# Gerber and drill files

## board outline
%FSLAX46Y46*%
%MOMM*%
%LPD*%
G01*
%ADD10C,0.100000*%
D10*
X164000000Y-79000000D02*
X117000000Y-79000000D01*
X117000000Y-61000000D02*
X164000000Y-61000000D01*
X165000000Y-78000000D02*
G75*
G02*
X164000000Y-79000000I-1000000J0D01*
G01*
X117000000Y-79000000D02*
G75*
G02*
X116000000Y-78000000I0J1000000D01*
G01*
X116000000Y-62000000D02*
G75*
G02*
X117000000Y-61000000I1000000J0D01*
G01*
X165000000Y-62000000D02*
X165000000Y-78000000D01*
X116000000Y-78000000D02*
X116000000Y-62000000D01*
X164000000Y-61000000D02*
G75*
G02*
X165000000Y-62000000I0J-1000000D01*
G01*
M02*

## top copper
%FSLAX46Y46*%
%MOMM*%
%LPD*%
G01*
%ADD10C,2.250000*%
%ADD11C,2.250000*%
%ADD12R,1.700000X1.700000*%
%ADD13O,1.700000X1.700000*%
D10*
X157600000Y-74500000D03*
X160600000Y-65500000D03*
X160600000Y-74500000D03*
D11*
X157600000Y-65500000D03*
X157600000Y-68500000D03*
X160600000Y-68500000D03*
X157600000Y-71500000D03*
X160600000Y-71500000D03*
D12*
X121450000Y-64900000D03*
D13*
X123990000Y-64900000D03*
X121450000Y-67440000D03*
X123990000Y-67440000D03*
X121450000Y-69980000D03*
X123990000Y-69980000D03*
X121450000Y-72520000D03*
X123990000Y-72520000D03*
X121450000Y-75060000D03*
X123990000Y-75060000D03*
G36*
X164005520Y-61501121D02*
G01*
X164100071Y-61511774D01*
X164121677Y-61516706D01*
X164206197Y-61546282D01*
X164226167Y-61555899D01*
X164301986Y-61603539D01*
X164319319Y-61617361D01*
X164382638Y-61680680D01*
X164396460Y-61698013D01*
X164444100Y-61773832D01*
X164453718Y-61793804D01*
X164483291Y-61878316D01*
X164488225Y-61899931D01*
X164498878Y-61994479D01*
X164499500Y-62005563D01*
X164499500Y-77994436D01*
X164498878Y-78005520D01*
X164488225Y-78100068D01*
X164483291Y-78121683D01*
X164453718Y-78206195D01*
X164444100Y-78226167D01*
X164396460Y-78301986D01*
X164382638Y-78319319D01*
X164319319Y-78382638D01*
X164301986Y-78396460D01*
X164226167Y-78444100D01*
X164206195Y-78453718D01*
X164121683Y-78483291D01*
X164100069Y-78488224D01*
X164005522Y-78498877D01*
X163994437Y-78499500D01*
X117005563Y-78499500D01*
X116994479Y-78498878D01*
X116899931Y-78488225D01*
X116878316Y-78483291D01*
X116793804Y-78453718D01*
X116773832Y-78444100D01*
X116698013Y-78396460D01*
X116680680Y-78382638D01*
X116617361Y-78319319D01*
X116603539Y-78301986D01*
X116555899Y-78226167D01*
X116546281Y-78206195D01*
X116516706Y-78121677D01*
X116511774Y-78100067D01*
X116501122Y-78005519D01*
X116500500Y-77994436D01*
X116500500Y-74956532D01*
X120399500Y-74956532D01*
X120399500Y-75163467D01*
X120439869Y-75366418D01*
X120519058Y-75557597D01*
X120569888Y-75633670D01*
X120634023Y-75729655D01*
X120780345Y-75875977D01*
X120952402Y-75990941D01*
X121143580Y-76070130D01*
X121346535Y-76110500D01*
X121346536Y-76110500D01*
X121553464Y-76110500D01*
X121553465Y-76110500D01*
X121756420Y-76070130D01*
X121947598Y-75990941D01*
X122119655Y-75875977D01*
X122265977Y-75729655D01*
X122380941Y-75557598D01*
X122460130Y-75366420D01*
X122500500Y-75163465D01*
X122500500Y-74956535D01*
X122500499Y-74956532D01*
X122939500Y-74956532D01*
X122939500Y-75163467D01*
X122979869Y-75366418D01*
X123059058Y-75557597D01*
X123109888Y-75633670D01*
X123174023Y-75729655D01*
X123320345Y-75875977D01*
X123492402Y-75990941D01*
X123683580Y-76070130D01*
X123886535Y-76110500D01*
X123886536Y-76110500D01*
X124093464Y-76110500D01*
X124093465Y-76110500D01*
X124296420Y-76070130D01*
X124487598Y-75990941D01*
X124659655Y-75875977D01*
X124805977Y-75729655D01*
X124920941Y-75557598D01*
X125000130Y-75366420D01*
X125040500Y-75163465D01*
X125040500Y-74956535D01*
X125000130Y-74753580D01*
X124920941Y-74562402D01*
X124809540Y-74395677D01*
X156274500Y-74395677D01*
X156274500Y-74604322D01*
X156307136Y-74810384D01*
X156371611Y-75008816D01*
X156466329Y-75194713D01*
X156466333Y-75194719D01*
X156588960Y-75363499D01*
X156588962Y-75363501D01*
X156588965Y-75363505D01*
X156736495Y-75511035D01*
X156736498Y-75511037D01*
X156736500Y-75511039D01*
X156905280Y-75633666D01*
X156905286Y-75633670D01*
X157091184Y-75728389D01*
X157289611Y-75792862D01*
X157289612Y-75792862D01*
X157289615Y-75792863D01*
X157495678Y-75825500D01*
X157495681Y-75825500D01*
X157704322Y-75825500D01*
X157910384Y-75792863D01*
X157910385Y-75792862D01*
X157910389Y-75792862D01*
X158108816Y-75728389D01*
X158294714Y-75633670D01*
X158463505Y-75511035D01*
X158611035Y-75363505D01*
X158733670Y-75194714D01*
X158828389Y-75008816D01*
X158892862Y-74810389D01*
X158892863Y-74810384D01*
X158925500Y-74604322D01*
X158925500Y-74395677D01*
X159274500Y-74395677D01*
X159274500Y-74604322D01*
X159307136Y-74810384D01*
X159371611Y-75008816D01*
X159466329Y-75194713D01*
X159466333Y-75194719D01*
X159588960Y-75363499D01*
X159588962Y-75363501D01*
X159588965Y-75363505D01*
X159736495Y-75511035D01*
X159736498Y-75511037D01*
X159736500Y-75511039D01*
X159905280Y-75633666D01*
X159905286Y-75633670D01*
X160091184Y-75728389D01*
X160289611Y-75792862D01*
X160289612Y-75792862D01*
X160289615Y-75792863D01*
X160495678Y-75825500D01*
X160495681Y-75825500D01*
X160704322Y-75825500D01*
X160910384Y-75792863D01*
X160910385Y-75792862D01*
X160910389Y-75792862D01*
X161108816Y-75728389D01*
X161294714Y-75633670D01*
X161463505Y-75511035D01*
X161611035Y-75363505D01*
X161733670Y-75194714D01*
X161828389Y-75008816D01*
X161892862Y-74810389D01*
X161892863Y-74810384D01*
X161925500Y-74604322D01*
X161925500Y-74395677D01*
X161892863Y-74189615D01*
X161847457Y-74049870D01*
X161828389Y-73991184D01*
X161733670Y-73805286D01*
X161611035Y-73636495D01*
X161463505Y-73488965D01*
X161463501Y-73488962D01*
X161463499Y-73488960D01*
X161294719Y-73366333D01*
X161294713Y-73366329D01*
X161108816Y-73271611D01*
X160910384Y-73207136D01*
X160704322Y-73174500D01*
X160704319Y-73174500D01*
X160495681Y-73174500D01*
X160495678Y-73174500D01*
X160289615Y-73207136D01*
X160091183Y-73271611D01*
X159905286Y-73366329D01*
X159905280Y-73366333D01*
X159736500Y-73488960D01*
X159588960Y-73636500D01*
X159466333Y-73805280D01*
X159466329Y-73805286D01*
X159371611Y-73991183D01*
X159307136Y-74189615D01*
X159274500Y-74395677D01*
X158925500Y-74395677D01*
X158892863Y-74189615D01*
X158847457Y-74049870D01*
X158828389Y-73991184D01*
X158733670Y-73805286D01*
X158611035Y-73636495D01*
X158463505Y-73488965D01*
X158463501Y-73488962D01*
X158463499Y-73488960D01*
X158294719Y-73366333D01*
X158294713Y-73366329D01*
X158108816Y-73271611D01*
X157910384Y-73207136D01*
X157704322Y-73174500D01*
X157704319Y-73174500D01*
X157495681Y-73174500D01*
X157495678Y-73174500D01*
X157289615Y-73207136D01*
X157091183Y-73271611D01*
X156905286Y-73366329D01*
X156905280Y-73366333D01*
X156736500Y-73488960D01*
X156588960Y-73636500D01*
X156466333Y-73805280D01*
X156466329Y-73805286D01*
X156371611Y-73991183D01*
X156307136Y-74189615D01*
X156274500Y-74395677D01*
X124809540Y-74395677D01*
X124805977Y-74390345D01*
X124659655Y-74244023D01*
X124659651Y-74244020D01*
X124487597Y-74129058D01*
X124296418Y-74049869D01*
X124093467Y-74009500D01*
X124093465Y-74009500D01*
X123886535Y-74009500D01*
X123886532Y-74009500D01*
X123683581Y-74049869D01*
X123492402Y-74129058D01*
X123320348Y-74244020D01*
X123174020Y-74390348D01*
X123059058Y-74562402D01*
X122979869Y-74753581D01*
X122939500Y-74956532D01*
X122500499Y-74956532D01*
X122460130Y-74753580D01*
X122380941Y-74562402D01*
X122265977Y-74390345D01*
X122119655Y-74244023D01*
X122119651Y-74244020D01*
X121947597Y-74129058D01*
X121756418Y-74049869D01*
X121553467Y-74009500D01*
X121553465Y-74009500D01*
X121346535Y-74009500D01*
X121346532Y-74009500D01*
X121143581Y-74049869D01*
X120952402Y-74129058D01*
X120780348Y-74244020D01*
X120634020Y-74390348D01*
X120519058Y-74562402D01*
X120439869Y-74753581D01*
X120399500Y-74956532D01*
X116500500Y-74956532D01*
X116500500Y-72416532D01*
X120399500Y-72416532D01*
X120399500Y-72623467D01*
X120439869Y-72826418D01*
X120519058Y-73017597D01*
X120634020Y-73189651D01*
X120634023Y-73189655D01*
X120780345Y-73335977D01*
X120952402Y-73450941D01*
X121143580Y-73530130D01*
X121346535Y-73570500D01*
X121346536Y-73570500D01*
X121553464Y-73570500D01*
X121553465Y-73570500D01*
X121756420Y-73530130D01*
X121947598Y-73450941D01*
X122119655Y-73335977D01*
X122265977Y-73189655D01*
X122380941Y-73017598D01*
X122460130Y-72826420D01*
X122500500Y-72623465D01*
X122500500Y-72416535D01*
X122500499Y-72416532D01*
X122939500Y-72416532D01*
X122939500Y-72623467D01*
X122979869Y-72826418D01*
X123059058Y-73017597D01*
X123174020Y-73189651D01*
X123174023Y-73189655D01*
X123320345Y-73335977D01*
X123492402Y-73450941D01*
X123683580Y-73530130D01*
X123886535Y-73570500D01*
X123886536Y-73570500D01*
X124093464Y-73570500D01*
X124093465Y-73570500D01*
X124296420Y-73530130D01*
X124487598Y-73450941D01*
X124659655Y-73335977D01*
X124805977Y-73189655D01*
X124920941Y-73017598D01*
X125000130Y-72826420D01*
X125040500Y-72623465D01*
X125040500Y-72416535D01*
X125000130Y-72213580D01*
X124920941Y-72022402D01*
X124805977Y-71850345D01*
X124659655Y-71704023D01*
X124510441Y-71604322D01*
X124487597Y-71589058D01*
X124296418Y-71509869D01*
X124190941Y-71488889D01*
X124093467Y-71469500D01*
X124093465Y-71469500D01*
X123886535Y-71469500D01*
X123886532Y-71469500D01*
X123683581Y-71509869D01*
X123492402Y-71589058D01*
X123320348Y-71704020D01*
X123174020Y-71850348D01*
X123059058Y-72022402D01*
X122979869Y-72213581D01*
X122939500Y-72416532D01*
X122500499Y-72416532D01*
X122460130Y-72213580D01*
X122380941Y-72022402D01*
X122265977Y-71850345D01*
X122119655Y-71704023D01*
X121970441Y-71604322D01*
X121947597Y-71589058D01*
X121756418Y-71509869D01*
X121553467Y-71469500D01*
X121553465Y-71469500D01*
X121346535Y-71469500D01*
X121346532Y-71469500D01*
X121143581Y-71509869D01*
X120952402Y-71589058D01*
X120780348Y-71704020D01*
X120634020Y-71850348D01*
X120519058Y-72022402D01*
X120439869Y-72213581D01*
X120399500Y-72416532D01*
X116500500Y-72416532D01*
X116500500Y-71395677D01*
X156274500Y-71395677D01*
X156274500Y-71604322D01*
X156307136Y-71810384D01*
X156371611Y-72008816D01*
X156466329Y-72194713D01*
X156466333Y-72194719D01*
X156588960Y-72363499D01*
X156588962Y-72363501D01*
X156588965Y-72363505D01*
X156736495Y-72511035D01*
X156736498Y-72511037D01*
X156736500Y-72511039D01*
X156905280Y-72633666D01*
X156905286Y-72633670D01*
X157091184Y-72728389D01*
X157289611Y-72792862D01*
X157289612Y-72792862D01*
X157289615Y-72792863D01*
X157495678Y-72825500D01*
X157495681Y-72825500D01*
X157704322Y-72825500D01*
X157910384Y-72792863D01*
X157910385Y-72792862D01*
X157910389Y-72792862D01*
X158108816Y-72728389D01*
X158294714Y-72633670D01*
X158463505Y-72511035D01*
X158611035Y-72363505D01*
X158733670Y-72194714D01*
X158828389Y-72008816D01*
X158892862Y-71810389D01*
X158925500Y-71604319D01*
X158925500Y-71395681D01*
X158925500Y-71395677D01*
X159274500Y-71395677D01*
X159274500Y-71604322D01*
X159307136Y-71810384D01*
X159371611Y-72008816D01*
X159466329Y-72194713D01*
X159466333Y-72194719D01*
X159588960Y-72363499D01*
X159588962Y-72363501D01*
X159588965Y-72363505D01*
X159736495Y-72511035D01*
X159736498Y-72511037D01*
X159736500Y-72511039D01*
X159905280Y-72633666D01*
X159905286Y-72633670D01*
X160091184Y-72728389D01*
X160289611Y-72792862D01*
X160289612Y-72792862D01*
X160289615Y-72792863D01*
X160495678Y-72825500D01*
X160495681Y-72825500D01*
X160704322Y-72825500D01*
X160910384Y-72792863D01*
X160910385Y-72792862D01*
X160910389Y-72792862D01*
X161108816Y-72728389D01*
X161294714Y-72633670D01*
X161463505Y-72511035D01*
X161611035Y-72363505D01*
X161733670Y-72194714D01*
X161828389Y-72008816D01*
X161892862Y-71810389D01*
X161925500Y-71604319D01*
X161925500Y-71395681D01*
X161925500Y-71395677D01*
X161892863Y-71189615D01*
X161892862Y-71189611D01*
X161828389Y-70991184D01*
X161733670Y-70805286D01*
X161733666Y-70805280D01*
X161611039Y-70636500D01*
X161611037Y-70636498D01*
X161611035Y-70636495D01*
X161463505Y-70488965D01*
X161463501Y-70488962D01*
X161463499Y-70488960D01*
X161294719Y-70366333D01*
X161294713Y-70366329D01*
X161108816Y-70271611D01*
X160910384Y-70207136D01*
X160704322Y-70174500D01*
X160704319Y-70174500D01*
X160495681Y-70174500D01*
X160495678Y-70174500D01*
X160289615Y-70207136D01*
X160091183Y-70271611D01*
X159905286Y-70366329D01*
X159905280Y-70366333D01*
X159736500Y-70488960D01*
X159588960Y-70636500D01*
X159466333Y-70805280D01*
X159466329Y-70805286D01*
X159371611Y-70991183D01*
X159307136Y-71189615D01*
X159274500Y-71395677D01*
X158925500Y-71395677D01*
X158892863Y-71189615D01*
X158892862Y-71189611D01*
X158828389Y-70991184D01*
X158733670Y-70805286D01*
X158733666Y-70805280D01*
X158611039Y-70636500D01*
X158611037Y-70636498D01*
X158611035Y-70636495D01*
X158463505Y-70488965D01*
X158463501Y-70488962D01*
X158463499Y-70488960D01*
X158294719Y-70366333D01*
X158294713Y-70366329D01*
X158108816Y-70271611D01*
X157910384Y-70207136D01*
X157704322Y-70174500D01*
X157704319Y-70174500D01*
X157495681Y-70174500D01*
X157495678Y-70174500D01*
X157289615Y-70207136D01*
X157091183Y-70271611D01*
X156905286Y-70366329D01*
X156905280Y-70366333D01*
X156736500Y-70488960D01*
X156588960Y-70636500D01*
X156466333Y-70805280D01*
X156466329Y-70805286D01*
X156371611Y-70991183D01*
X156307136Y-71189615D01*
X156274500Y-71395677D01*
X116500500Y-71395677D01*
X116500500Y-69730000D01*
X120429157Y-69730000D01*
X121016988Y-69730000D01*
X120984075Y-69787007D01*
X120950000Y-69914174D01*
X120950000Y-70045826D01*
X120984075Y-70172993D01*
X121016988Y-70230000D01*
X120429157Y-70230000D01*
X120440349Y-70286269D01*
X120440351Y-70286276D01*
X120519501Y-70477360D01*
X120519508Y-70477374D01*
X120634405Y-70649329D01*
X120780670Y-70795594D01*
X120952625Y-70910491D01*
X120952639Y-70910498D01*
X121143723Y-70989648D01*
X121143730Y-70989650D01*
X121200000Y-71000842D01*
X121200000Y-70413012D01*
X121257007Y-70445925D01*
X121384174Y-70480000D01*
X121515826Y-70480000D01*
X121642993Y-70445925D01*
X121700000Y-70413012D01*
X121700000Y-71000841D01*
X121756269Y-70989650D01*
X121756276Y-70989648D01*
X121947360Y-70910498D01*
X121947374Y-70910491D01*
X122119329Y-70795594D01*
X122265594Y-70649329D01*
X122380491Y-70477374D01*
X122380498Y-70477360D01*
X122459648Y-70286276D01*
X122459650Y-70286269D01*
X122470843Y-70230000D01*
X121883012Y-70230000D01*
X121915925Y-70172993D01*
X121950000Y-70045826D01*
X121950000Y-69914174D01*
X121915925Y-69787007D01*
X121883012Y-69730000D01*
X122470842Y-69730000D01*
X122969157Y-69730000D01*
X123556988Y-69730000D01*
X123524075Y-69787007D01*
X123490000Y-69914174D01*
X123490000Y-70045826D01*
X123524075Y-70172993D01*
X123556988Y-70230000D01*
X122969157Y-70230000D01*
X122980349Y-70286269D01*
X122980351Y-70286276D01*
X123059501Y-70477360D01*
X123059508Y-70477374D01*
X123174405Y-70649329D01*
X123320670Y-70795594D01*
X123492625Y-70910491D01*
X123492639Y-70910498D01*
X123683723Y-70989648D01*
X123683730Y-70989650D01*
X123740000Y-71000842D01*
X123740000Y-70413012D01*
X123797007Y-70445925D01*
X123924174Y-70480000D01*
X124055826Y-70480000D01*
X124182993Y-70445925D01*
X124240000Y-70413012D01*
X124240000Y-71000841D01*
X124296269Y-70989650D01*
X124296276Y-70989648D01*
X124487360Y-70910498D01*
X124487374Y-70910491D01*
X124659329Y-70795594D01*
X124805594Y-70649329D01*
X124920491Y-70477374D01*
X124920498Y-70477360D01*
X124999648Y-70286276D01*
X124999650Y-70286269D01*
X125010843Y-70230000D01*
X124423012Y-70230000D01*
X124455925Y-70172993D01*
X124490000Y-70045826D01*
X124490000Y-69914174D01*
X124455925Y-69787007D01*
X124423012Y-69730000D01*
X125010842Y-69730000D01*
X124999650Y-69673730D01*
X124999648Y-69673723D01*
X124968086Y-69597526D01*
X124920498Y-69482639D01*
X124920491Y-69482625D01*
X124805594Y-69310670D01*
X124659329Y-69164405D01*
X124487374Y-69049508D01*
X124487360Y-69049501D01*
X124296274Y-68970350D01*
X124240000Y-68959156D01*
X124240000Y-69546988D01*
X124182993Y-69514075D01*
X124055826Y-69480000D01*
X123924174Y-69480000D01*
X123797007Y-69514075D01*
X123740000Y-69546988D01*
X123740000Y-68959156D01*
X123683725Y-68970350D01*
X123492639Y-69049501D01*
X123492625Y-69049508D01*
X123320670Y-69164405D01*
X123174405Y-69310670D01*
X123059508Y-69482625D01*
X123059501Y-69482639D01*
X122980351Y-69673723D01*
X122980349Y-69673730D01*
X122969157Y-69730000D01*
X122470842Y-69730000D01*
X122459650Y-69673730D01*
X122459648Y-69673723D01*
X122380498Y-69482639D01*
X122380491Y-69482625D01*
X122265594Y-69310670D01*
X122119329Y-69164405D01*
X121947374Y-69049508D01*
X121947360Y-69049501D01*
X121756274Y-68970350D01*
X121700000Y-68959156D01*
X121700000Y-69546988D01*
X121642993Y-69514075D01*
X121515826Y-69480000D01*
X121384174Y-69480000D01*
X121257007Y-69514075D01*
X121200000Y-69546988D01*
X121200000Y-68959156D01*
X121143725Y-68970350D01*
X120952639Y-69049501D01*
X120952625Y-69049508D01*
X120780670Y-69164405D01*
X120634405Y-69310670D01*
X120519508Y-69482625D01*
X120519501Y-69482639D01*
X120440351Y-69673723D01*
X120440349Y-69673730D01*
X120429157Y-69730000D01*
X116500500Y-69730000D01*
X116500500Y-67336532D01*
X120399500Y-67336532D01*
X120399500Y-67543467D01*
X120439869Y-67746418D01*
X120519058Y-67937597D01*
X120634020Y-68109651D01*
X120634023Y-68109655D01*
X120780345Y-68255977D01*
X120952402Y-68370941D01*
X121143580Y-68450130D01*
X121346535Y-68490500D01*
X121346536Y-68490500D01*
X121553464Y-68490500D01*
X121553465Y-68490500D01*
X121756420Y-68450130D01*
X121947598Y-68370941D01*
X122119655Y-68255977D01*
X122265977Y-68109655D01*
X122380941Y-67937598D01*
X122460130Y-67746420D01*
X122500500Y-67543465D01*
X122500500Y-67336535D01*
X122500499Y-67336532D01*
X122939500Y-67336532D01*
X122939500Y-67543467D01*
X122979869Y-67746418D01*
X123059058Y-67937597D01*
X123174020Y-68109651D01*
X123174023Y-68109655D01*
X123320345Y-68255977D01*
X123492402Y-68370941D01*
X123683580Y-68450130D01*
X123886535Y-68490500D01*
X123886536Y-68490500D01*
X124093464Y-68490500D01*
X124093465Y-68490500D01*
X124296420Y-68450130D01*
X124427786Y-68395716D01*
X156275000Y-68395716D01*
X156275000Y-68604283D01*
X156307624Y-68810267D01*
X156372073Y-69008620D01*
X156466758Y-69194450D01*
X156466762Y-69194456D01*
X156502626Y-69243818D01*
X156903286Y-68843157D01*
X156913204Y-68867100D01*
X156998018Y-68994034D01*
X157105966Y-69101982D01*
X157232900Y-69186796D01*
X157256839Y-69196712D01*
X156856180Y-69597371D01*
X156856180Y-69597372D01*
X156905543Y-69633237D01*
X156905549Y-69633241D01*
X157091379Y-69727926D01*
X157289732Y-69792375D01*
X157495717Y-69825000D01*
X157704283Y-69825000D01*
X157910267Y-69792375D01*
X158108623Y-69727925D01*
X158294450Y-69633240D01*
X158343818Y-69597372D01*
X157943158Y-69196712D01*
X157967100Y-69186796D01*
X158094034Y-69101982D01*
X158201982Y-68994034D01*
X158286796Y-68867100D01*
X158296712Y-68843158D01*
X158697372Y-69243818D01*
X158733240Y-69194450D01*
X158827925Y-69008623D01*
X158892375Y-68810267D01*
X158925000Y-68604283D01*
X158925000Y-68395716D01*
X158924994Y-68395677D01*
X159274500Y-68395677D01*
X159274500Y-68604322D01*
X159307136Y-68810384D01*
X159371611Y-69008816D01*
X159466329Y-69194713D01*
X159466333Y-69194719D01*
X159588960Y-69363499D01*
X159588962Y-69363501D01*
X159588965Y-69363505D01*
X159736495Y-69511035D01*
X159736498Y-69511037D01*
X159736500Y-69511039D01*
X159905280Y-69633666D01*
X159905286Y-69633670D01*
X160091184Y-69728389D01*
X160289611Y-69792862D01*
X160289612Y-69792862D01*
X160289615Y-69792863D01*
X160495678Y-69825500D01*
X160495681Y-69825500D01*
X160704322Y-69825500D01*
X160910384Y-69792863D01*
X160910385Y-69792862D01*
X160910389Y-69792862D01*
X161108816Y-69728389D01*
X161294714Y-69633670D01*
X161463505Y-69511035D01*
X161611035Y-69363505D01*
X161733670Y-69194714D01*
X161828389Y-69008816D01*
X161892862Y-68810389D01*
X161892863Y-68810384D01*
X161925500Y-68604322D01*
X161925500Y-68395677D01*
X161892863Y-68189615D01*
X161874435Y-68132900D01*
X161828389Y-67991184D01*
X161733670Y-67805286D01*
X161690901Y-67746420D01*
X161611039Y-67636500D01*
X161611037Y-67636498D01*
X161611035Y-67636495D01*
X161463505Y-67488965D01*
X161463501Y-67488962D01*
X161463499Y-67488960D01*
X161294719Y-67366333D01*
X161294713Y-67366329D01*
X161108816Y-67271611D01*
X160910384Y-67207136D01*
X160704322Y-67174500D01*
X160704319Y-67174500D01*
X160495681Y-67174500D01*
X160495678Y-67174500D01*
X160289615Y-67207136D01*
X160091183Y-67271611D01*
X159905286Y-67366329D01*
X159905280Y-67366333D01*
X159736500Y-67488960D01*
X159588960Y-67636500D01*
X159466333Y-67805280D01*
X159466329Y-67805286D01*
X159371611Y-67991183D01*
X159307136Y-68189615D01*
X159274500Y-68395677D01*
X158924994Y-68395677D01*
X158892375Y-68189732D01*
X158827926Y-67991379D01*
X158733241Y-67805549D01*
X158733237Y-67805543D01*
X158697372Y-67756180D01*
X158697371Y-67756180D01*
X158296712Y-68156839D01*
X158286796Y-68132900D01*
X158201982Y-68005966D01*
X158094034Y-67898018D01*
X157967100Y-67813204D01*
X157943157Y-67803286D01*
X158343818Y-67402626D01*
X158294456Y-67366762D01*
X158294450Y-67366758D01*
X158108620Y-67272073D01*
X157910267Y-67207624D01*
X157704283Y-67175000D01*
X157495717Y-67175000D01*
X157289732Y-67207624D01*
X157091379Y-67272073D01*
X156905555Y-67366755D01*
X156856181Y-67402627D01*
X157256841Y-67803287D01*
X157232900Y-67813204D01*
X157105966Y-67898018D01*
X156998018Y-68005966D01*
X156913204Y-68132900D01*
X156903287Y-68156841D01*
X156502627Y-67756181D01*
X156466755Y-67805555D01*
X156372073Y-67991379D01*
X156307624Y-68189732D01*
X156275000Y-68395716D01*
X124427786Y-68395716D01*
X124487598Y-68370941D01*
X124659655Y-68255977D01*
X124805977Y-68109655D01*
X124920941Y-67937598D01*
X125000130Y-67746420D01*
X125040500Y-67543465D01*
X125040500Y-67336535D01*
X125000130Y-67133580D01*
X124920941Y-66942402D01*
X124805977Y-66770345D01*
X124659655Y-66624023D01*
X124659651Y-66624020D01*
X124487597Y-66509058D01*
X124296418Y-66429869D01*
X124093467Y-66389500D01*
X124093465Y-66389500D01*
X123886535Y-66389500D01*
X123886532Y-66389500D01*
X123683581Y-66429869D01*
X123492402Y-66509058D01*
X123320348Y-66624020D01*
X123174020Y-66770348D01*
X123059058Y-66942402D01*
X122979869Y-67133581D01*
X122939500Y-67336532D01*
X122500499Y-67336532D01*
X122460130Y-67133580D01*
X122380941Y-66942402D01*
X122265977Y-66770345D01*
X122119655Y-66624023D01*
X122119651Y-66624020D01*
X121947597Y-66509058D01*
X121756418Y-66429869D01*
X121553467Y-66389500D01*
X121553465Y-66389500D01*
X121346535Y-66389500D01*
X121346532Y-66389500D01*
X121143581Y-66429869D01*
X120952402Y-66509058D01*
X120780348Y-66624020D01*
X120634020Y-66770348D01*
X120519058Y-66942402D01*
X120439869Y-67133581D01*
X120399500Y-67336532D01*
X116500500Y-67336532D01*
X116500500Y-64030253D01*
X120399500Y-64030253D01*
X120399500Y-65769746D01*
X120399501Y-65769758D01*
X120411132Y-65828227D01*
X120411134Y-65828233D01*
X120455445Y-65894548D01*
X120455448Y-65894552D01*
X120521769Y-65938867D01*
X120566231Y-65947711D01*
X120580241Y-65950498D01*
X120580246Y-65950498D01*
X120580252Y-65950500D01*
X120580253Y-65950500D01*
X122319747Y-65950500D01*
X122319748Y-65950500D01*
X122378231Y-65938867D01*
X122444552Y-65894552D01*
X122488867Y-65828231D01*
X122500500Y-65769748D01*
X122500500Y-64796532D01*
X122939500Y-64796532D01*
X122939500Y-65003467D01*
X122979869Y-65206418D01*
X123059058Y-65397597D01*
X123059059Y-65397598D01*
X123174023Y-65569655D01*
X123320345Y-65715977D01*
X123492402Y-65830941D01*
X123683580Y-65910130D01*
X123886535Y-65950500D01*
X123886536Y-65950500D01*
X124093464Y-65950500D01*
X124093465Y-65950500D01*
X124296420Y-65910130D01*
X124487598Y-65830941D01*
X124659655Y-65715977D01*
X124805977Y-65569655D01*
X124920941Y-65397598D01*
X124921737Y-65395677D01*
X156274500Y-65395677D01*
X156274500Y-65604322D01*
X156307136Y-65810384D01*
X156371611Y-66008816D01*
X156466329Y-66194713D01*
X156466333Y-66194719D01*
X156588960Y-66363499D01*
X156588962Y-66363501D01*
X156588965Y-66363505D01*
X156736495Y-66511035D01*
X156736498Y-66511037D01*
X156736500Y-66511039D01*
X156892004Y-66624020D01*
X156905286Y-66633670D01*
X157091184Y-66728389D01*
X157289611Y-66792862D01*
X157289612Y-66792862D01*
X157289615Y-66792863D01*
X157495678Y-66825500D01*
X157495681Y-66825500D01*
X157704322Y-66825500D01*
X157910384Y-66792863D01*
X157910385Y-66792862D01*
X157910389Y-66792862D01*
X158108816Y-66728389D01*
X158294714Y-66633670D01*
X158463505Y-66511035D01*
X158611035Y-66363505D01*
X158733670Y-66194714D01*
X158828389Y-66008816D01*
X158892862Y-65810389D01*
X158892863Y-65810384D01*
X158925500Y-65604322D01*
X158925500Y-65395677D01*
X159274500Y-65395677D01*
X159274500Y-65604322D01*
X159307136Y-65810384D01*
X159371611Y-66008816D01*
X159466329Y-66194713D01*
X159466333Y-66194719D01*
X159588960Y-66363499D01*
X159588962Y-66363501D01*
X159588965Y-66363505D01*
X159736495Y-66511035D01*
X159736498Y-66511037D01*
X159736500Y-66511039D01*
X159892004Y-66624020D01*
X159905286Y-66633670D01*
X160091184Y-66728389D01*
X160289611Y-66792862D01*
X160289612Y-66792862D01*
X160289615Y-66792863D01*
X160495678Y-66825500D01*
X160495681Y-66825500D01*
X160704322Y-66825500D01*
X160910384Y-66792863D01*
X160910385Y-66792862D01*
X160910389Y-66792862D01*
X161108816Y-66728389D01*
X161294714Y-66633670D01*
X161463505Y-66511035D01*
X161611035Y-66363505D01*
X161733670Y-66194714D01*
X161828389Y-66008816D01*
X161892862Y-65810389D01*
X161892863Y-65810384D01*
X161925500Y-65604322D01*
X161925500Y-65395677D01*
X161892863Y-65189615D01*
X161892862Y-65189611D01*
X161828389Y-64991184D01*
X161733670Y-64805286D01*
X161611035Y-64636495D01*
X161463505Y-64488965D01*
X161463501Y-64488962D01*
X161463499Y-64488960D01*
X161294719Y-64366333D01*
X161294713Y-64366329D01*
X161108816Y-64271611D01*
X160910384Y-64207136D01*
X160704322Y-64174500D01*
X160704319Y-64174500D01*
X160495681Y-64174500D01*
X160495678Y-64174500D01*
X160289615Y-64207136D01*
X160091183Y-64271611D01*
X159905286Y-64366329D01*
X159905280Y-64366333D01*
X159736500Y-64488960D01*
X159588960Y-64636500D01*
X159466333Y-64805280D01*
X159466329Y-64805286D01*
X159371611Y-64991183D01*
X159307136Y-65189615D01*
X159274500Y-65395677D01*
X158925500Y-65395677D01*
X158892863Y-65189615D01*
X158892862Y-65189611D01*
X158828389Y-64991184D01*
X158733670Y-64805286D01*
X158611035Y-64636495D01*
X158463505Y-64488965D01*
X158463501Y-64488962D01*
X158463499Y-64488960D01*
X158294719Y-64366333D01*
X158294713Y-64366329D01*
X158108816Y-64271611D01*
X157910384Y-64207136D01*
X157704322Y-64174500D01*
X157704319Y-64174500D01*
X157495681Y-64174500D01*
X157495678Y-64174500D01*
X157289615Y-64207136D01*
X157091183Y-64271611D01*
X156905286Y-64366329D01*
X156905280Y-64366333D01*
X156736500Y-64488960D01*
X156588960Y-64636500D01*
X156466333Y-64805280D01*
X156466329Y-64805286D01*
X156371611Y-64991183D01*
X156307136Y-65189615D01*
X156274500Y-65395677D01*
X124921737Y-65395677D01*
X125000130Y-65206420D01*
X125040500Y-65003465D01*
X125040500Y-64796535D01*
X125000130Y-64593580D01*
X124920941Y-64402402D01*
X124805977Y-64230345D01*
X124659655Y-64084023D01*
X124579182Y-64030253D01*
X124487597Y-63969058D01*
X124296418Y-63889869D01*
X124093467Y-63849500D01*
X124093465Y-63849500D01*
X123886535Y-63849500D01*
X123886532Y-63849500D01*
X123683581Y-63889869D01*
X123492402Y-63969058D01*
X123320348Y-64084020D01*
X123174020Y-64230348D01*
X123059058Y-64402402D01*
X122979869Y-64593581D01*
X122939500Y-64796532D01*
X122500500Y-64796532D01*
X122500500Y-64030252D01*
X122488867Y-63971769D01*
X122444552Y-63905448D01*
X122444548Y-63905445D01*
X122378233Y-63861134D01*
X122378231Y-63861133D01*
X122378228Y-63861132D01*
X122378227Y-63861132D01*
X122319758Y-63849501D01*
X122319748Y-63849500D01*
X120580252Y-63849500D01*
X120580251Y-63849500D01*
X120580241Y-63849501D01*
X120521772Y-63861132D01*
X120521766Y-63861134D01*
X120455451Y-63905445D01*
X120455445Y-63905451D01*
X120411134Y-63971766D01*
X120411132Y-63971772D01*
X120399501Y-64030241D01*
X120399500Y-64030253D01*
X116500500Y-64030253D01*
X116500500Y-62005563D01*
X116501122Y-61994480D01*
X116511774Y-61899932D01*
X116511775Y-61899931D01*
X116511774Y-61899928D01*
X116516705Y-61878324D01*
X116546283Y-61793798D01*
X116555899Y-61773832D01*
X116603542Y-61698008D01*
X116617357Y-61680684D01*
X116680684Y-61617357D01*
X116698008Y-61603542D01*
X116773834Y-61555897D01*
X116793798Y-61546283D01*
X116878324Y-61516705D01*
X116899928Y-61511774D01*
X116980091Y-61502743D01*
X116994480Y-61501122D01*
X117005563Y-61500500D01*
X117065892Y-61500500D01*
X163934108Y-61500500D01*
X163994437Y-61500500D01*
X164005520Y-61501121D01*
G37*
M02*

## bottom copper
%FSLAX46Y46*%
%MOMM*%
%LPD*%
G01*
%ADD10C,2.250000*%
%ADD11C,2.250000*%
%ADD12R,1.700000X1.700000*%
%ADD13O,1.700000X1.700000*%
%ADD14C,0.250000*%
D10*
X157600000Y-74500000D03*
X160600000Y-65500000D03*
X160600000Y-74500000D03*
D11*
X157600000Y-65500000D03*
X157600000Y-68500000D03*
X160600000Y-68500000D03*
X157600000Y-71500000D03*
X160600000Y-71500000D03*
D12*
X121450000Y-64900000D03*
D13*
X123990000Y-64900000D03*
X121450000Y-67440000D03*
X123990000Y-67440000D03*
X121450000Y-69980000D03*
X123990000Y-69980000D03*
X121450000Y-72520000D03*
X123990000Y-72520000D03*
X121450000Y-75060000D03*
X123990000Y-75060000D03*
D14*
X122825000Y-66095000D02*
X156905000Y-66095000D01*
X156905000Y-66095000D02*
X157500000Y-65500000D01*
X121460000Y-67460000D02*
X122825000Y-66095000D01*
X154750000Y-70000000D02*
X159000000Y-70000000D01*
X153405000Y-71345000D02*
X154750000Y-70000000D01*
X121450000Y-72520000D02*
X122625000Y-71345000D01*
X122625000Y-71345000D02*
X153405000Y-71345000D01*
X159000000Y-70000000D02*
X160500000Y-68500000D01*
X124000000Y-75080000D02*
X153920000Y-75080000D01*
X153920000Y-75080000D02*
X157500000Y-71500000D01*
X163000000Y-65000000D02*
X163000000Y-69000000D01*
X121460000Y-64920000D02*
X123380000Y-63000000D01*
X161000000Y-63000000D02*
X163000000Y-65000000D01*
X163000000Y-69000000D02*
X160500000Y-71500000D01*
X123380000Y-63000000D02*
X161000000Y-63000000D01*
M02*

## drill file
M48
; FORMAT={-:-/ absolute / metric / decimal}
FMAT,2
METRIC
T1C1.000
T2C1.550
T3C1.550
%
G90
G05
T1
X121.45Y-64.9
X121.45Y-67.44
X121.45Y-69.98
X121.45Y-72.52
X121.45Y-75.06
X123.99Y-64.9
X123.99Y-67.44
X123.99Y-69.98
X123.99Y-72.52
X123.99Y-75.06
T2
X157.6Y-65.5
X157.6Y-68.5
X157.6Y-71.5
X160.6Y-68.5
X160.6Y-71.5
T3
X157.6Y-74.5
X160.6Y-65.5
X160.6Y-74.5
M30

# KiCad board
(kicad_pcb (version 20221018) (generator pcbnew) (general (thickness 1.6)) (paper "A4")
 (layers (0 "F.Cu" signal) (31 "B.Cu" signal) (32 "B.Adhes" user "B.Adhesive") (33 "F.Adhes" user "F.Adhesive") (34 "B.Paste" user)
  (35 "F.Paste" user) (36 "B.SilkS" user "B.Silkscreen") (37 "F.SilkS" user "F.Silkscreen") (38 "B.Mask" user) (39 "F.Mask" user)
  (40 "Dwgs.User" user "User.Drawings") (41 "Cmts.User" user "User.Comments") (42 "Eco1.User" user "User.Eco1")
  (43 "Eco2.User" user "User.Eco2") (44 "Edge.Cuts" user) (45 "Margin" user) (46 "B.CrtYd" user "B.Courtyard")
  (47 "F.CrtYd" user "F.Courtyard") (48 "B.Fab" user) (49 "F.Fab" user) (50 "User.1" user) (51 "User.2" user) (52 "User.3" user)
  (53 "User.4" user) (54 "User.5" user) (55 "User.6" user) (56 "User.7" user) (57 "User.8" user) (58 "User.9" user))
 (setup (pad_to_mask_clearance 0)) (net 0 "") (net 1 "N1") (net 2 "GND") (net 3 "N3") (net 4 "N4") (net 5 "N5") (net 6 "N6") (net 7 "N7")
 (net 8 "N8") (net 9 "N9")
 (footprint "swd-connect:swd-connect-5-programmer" (layer "F.Cu") (at 159.1 70)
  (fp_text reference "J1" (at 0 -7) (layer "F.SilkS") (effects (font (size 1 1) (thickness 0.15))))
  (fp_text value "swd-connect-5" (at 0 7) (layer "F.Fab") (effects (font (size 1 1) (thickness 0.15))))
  (pad "" np_thru_hole circle (at -1.5 4.5) (size 2.25 2.25) (drill 1.55) (layers "F&B.Cu" "*.Mask"))
  (pad "" np_thru_hole circle (at 1.5 -4.5) (size 2.25 2.25) (drill 1.55) (layers "F&B.Cu" "*.Mask"))
  (pad "" np_thru_hole circle (at 1.5 4.5) (size 2.25 2.25) (drill 1.55) (layers "F&B.Cu" "*.Mask"))
  (pad "1" thru_hole circle (at -1.5 -4.5) (size 2.25 2.25) (drill 1.55) (layers "*.Cu" "*.Mask") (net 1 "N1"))
  (pad "2" thru_hole circle (at -1.5 -1.5) (size 2.25 2.25) (drill 1.55) (layers "*.Cu" "*.Mask") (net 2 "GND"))
  (pad "3" thru_hole circle (at 1.5 -1.5) (size 2.25 2.25) (drill 1.55) (layers "*.Cu" "*.Mask") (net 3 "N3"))
  (pad "4" thru_hole circle (at -1.5 1.5) (size 2.25 2.25) (drill 1.55) (layers "*.Cu" "*.Mask") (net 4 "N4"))
  (pad "5" thru_hole circle (at 1.5 1.5) (size 2.25 2.25) (drill 1.55) (layers "*.Cu" "*.Mask") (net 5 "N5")))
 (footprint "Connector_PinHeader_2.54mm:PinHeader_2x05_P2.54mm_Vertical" (layer "F.Cu") (at 121.45 64.9)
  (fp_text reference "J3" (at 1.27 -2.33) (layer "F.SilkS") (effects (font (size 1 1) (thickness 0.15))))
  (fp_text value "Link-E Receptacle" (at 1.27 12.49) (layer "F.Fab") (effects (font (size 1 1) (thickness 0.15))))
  (pad "1" thru_hole rect (at 0 0) (size 1.7 1.7) (drill 1) (layers "*.Cu" "*.Mask") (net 5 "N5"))
  (pad "2" thru_hole oval (at 2.54 0) (size 1.7 1.7) (drill 1) (layers "*.Cu" "*.Mask") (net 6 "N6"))
  (pad "3" thru_hole oval (at 0 2.54) (size 1.7 1.7) (drill 1) (layers "*.Cu" "*.Mask") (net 1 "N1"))
  (pad "4" thru_hole oval (at 2.54 2.54) (size 1.7 1.7) (drill 1) (layers "*.Cu" "*.Mask") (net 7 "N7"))
  (pad "5" thru_hole oval (at 0 5.08) (size 1.7 1.7) (drill 1) (layers "*.Cu" "*.Mask") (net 2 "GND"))
  (pad "6" thru_hole oval (at 2.54 5.08) (size 1.7 1.7) (drill 1) (layers "*.Cu" "*.Mask") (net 2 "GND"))
  (pad "7" thru_hole oval (at 0 7.62) (size 1.7 1.7) (drill 1) (layers "*.Cu" "*.Mask") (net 3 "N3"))
  (pad "8" thru_hole oval (at 2.54 7.62) (size 1.7 1.7) (drill 1) (layers "*.Cu" "*.Mask") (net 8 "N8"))
  (pad "9" thru_hole oval (at 0 10.16) (size 1.7 1.7) (drill 1) (layers "*.Cu" "*.Mask") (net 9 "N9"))
  (pad "10" thru_hole oval (at 2.54 10.16) (size 1.7 1.7) (drill 1) (layers "*.Cu" "*.Mask") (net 4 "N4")))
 (gr_line (start 164 79) (end 117 79) (stroke (width 0.1) (type default)) (layer "Edge.Cuts"))
 (gr_line (start 117 61) (end 164 61) (stroke (width 0.1) (type default)) (layer "Edge.Cuts"))
 (gr_arc (start 165 78) (mid 164.707107 78.707107) (end 164 79) (stroke (width 0.1) (type default)) (layer "Edge.Cuts"))
 (gr_arc (start 117 79) (mid 116.292893 78.707107) (end 116 78) (stroke (width 0.1) (type default)) (layer "Edge.Cuts"))
 (gr_arc (start 116 62) (mid 116.292893 61.292893) (end 117 61) (stroke (width 0.1) (type default)) (layer "Edge.Cuts"))
 (gr_line (start 165 62) (end 165 78) (stroke (width 0.1) (type default)) (layer "Edge.Cuts"))
 (gr_line (start 116 78) (end 116 62) (stroke (width 0.1) (type default)) (layer "Edge.Cuts"))
 (gr_arc (start 164 61) (mid 164.707107 61.292893) (end 165 62) (stroke (width 0.1) (type default)) (layer "Edge.Cuts"))
 (segment (start 122.825 66.095) (end 156.905 66.095) (width 0.25) (layer "B.Cu") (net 1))
 (segment (start 156.905 66.095) (end 157.5 65.5) (width 0.25) (layer "B.Cu") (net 1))
 (segment (start 121.46 67.46) (end 122.825 66.095) (width 0.25) (layer "B.Cu") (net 1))
 (segment (start 154.75 70) (end 159 70) (width 0.25) (layer "B.Cu") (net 3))
 (segment (start 153.405 71.345) (end 154.75 70) (width 0.25) (layer "B.Cu") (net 3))
 (segment (start 121.45 72.52) (end 122.625 71.345) (width 0.25) (layer "B.Cu") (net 3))
 (segment (start 122.625 71.345) (end 153.405 71.345) (width 0.25) (layer "B.Cu") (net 3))
 (segment (start 159 70) (end 160.5 68.5) (width 0.25) (layer "B.Cu") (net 3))
 (segment (start 124 75.08) (end 153.92 75.08) (width 0.25) (layer "B.Cu") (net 4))
 (segment (start 153.92 75.08) (end 157.5 71.5) (width 0.25) (layer "B.Cu") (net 4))
 (segment (start 163 65) (end 163 69) (width 0.25) (layer "B.Cu") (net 5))
 (segment (start 121.46 64.92) (end 123.38 63) (width 0.25) (layer "B.Cu") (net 5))
 (segment (start 161 63) (end 163 65) (width 0.25) (layer "B.Cu") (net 5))
 (segment (start 163 69) (end 160.5 71.5) (width 0.25) (layer "B.Cu") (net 5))
 (segment (start 123.38 63) (end 161 63) (width 0.25) (layer "B.Cu") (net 5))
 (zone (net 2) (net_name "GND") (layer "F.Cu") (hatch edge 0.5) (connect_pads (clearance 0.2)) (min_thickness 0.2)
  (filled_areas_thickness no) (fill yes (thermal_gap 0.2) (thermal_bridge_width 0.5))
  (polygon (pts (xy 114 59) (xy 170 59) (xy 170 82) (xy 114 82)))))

